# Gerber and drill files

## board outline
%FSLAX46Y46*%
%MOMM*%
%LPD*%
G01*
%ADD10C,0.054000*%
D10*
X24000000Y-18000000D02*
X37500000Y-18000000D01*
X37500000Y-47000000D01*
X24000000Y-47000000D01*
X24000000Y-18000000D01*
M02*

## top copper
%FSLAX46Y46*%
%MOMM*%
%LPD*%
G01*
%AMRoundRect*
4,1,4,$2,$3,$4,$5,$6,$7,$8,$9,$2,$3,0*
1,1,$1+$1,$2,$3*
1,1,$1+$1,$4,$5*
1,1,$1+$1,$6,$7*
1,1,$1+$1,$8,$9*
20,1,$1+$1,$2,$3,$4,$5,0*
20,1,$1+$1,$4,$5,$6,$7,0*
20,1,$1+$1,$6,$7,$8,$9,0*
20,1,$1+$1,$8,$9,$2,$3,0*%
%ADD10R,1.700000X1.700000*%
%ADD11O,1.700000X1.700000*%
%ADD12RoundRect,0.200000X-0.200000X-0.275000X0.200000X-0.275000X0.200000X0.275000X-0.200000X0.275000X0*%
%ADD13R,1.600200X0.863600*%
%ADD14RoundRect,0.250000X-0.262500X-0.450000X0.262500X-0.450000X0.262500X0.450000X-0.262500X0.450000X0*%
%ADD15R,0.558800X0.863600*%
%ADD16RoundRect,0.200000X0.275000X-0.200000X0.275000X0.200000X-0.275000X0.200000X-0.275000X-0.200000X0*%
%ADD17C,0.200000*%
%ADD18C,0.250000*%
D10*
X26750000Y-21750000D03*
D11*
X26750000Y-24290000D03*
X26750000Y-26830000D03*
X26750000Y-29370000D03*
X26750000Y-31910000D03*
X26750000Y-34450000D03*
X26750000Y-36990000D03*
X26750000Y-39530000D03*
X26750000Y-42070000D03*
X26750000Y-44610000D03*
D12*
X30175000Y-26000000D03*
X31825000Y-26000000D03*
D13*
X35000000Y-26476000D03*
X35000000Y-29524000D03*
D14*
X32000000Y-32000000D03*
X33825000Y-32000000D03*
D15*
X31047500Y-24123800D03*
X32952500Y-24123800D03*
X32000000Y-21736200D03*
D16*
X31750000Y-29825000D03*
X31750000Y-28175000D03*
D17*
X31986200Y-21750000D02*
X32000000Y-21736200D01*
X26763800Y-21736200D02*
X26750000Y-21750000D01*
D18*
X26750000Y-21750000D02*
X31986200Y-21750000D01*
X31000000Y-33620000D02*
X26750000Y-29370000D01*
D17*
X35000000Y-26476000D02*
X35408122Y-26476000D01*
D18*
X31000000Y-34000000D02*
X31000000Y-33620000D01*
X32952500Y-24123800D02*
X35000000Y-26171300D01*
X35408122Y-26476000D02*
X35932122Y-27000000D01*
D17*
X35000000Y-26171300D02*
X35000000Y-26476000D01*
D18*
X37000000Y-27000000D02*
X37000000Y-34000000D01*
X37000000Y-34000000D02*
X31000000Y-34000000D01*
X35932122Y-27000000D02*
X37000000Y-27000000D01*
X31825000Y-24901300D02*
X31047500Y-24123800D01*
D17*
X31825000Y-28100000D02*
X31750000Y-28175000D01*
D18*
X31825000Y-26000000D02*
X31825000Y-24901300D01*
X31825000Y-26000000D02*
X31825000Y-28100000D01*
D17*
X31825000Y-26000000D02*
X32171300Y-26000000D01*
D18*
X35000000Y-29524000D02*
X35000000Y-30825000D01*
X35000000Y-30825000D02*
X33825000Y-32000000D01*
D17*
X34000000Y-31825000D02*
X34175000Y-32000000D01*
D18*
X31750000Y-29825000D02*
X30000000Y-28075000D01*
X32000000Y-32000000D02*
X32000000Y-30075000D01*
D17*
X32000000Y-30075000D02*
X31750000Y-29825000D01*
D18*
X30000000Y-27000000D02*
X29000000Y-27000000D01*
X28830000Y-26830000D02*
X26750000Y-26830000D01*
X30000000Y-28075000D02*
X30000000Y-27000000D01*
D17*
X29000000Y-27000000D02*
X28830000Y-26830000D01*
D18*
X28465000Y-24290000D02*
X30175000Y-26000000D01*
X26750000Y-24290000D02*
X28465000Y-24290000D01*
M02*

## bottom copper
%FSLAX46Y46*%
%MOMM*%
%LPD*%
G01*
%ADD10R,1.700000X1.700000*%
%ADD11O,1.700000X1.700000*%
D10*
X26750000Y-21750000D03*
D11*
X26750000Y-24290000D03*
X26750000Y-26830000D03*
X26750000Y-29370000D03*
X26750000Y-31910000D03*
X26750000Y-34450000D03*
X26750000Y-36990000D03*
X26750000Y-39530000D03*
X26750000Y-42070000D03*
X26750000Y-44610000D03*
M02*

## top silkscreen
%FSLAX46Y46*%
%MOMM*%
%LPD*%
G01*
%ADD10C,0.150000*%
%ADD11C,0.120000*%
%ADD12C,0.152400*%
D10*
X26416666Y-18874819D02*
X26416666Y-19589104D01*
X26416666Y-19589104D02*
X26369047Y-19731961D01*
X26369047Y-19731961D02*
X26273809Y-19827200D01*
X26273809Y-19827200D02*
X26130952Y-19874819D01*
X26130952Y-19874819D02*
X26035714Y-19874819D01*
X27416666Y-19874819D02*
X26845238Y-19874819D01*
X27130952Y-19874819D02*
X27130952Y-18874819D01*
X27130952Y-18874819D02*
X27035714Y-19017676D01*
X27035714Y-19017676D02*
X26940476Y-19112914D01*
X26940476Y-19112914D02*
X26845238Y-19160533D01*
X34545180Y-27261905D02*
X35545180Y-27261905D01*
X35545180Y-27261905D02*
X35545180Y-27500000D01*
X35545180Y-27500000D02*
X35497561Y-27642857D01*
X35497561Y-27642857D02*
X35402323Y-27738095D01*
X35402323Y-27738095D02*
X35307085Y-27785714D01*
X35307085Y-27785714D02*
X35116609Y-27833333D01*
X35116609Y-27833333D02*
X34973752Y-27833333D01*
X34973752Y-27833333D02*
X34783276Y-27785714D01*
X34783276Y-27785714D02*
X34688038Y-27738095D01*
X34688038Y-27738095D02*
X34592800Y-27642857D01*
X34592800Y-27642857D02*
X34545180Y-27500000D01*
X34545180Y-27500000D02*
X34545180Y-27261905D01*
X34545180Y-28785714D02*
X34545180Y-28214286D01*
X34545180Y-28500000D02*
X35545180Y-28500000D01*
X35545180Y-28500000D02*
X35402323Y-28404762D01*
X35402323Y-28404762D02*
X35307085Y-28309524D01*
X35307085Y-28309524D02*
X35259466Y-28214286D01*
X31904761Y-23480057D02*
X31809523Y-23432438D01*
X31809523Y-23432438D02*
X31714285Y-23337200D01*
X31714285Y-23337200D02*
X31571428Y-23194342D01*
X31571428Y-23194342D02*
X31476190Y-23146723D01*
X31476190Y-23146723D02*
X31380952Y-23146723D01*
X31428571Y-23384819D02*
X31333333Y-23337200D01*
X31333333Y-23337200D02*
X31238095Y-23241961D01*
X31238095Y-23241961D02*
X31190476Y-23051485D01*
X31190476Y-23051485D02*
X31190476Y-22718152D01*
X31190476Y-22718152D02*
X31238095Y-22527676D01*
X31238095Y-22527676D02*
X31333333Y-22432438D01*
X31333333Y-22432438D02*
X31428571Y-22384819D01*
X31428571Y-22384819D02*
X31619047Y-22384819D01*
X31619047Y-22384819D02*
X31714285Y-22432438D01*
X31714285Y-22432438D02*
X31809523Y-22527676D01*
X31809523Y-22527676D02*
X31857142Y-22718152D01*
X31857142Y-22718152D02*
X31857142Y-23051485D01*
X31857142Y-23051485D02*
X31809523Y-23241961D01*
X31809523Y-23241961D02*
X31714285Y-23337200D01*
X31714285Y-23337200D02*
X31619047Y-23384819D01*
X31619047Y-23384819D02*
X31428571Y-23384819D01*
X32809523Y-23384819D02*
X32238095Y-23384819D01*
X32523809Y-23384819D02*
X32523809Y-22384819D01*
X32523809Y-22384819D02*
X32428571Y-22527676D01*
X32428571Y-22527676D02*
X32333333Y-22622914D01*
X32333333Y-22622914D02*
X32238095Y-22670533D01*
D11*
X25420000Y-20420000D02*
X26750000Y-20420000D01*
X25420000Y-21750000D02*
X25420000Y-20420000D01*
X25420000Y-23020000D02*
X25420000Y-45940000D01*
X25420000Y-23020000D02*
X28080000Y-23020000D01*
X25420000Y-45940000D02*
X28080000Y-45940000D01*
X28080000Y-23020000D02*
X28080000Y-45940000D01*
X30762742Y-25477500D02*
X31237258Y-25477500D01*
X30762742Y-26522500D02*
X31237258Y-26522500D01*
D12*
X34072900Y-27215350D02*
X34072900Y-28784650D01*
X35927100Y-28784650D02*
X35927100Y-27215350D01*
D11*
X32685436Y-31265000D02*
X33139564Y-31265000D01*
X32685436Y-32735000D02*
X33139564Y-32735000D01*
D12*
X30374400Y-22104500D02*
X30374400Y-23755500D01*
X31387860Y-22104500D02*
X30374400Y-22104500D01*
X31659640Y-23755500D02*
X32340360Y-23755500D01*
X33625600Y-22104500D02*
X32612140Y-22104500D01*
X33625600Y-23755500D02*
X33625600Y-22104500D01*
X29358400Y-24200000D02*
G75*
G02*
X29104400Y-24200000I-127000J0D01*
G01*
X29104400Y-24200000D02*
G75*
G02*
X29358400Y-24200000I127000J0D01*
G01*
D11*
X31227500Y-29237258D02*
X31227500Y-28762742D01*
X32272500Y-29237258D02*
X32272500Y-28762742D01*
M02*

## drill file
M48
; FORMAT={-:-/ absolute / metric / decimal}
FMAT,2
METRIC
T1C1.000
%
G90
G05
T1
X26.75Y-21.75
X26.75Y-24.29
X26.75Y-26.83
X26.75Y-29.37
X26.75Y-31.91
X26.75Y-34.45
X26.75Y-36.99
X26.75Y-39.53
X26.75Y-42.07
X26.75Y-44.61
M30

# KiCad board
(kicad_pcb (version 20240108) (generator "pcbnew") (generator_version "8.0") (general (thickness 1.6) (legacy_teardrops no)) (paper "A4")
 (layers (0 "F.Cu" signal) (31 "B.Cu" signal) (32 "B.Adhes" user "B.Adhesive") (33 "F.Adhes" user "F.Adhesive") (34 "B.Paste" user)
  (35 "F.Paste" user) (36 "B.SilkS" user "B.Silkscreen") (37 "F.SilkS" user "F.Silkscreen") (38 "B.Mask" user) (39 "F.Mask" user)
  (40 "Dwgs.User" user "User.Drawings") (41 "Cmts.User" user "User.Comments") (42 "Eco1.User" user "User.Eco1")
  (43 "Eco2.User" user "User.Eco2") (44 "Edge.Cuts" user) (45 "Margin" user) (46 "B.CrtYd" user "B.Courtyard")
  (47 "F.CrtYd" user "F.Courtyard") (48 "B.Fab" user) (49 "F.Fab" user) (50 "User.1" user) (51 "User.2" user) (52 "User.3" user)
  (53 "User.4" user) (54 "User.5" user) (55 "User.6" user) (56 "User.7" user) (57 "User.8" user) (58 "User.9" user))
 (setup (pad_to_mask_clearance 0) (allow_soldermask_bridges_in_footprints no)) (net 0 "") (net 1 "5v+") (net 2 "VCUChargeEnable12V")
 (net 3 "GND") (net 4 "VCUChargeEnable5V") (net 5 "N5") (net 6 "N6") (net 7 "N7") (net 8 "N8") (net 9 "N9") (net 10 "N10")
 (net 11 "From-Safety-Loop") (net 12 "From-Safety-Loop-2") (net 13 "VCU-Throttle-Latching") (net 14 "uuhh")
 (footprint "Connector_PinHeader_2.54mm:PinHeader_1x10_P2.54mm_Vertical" (layer "F.Cu") (at 26.75 21.75)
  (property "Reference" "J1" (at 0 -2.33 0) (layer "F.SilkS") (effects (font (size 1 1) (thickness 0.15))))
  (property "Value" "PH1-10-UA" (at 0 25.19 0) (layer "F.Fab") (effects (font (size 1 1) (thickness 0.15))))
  (fp_line (start -1.33 -1.33) (end 0 -1.33) (stroke (width 0.12) (type solid)) (layer "F.SilkS"))
  (fp_line (start -1.33 0) (end -1.33 -1.33) (stroke (width 0.12) (type solid)) (layer "F.SilkS"))
  (fp_line (start -1.33 1.27) (end -1.33 24.19) (stroke (width 0.12) (type solid)) (layer "F.SilkS"))
  (fp_line (start -1.33 1.27) (end 1.33 1.27) (stroke (width 0.12) (type solid)) (layer "F.SilkS"))
  (fp_line (start -1.33 24.19) (end 1.33 24.19) (stroke (width 0.12) (type solid)) (layer "F.SilkS"))
  (fp_line (start 1.33 1.27) (end 1.33 24.19) (stroke (width 0.12) (type solid)) (layer "F.SilkS"))
  (pad "1" thru_hole rect (at 0 0) (size 1.7 1.7) (drill 1) (layers "*.Cu" "*.Mask") (remove_unused_layers no) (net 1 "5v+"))
  (pad "2" thru_hole oval (at 0 2.54) (size 1.7 1.7) (drill 1) (layers "*.Cu" "*.Mask") (remove_unused_layers no)
   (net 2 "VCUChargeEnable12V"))
  (pad "3" thru_hole oval (at 0 5.08) (size 1.7 1.7) (drill 1) (layers "*.Cu" "*.Mask") (remove_unused_layers no) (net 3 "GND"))
  (pad "4" thru_hole oval (at 0 7.62) (size 1.7 1.7) (drill 1) (layers "*.Cu" "*.Mask") (remove_unused_layers no)
   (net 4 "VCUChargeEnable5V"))
  (pad "5" thru_hole oval (at 0 10.16) (size 1.7 1.7) (drill 1) (layers "*.Cu" "*.Mask") (remove_unused_layers no) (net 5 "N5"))
  (pad "6" thru_hole oval (at 0 12.7) (size 1.7 1.7) (drill 1) (layers "*.Cu" "*.Mask") (remove_unused_layers no) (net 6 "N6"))
  (pad "7" thru_hole oval (at 0 15.24) (size 1.7 1.7) (drill 1) (layers "*.Cu" "*.Mask") (remove_unused_layers no) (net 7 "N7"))
  (pad "8" thru_hole oval (at 0 17.78) (size 1.7 1.7) (drill 1) (layers "*.Cu" "*.Mask") (remove_unused_layers no) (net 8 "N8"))
  (pad "9" thru_hole oval (at 0 20.32) (size 1.7 1.7) (drill 1) (layers "*.Cu" "*.Mask") (remove_unused_layers no) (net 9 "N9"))
  (pad "10" thru_hole oval (at 0 22.86) (size 1.7 1.7) (drill 1) (layers "*.Cu" "*.Mask") (remove_unused_layers no) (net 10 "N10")))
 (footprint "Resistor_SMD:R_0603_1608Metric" (layer "F.Cu") (at 31 26)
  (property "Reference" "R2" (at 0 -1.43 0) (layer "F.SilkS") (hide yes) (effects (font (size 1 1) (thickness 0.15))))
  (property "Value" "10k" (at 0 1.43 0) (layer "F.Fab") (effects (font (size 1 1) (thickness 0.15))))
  (fp_line (start -0.237258 -0.5225) (end 0.237258 -0.5225) (stroke (width 0.12) (type solid)) (layer "F.SilkS"))
  (fp_line (start -0.237258 0.5225) (end 0.237258 0.5225) (stroke (width 0.12) (type solid)) (layer "F.SilkS"))
  (pad "1" smd roundrect (at -0.825 0) (size 0.8 0.95) (layers "F.Cu" "F.Paste" "F.Mask") (roundrect_rratio 0.25)
   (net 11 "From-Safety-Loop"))
  (pad "2" smd roundrect (at 0.825 0) (size 0.8 0.95) (layers "F.Cu" "F.Paste" "F.Mask") (roundrect_rratio 0.25)
   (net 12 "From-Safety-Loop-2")))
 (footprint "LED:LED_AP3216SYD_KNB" (layer "F.Cu") (at 35 28 -90)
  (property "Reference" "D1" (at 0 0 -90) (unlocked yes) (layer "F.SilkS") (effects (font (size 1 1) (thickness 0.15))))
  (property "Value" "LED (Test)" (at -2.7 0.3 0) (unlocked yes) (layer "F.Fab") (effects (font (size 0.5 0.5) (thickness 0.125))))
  (fp_line (start -0.78465 0.9271) (end 0.78465 0.9271) (stroke (width 0.1524) (type solid)) (layer "F.SilkS"))
  (fp_line (start 0.78465 -0.9271) (end -0.78465 -0.9271) (stroke (width 0.1524) (type solid)) (layer "F.SilkS"))
  (pad "1" smd rect (at -1.524 0 270) (size 0.8636 1.6002) (layers "F.Cu" "F.Paste" "F.Mask") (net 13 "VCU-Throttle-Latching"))
  (pad "2" smd rect (at 1.524 0 270) (size 0.8636 1.6002) (layers "F.Cu" "F.Paste" "F.Mask") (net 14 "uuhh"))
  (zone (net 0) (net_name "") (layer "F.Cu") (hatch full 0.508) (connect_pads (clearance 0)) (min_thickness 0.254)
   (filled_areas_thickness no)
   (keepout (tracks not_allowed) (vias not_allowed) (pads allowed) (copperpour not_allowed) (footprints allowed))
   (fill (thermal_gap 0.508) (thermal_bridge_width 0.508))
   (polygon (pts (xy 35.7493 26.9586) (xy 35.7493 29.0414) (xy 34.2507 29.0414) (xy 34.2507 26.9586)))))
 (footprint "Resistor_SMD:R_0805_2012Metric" (layer "F.Cu") (at 32.9125 32)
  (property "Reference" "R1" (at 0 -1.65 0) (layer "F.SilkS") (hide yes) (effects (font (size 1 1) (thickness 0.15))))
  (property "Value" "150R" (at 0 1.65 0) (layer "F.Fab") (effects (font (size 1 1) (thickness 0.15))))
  (fp_line (start -0.227064 -0.735) (end 0.227064 -0.735) (stroke (width 0.12) (type solid)) (layer "F.SilkS"))
  (fp_line (start -0.227064 0.735) (end 0.227064 0.735) (stroke (width 0.12) (type solid)) (layer "F.SilkS"))
  (pad "1" smd roundrect (at -0.9125 0) (size 1.025 1.4) (layers "F.Cu" "F.Paste" "F.Mask") (roundrect_rratio 0.243902) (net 3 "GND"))
  (pad "2" smd roundrect (at 0.9125 0) (size 1.025 1.4) (layers "F.Cu" "F.Paste" "F.Mask") (roundrect_rratio 0.243902) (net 14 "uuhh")))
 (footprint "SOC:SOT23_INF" (layer "F.Cu") (at 32 22.93)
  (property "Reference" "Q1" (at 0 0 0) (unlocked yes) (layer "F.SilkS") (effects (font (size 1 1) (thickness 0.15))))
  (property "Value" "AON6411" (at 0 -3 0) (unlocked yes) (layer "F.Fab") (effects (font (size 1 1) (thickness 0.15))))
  (fp_line (start -1.6256 -0.8255) (end -1.6256 0.8255) (stroke (width 0.1524) (type solid)) (layer "F.SilkS"))
  (fp_line (start -0.61214 -0.8255) (end -1.6256 -0.8255) (stroke (width 0.1524) (type solid)) (layer "F.SilkS"))
  (fp_line (start -0.34036 0.8255) (end 0.34036 0.8255) (stroke (width 0.1524) (type solid)) (layer "F.SilkS"))
  (fp_line (start 1.6256 -0.8255) (end 0.61214 -0.8255) (stroke (width 0.1524) (type solid)) (layer "F.SilkS"))
  (fp_line (start 1.6256 0.8255) (end 1.6256 -0.8255) (stroke (width 0.1524) (type solid)) (layer "F.SilkS"))
  (fp_circle (center -2.7686 1.27) (end -2.6416 1.27) (stroke (width 0.1524) (type solid)) (fill none) (layer "F.SilkS"))
  (pad "1" smd rect (at -0.9525 1.1938) (size 0.5588 0.8636) (layers "F.Cu" "F.Paste" "F.Mask") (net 12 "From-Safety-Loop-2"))
  (pad "2" smd rect (at 0.9525 1.1938) (size 0.5588 0.8636) (layers "F.Cu" "F.Paste" "F.Mask") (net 13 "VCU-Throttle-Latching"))
  (pad "3" smd rect (at 0 -1.1938) (size 0.5588 0.8636) (layers "F.Cu" "F.Paste" "F.Mask") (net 1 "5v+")))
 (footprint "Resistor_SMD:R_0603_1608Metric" (layer "F.Cu") (at 31.75 29 90)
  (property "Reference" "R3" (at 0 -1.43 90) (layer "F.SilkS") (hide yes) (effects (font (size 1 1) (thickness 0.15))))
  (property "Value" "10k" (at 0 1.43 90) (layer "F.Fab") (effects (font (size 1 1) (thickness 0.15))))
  (fp_line (start -0.237258 -0.5225) (end 0.237258 -0.5225) (stroke (width 0.12) (type solid)) (layer "F.SilkS"))
  (fp_line (start -0.237258 0.5225) (end 0.237258 0.5225) (stroke (width 0.12) (type solid)) (layer "F.SilkS"))
  (pad "1" smd roundrect (at -0.825 0 90) (size 0.8 0.95) (layers "F.Cu" "F.Paste" "F.Mask") (roundrect_rratio 0.25) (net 3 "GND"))
  (pad "2" smd roundrect (at 0.825 0 90) (size 0.8 0.95) (layers "F.Cu" "F.Paste" "F.Mask") (roundrect_rratio 0.25)
   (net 12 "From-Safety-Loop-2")))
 (gr_rect (start 24 18) (end 37.5 47) (stroke (width 0.054) (type default)) (fill none) (layer "Edge.Cuts"))
 (segment (start 31.9862 21.75) (end 32 21.7362) (width 0.2) (layer "F.Cu") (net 1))
 (segment (start 26.7638 21.7362) (end 26.75 21.75) (width 0.2) (layer "F.Cu") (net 1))
 (segment (start 26.75 21.75) (end 31.9862 21.75) (width 0.25) (layer "F.Cu") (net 1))
 (segment (start 31 33.62) (end 26.75 29.37) (width 0.25) (layer "F.Cu") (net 13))
 (segment (start 35 26.476) (end 35.408122 26.476) (width 0.2) (layer "F.Cu") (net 13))
 (segment (start 31 34) (end 31 33.62) (width 0.25) (layer "F.Cu") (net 13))
 (segment (start 32.9525 24.1238) (end 35 26.1713) (width 0.25) (layer "F.Cu") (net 13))
 (segment (start 35.408122 26.476) (end 35.932122 27) (width 0.25) (layer "F.Cu") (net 13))
 (segment (start 35 26.1713) (end 35 26.476) (width 0.2) (layer "F.Cu") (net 13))
 (segment (start 37 27) (end 37 34) (width 0.25) (layer "F.Cu") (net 13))
 (segment (start 37 34) (end 31 34) (width 0.25) (layer "F.Cu") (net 13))
 (segment (start 35.932122 27) (end 37 27) (width 0.25) (layer "F.Cu") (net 13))
 (segment (start 31.825 24.9013) (end 31.0475 24.1238) (width 0.25) (layer "F.Cu") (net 12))
 (segment (start 31.825 28.1) (end 31.75 28.175) (width 0.2) (layer "F.Cu") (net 12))
 (segment (start 31.825 26) (end 31.825 24.9013) (width 0.25) (layer "F.Cu") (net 12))
 (segment (start 31.825 26) (end 31.825 28.1) (width 0.25) (layer "F.Cu") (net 12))
 (segment (start 31.825 26) (end 32.1713 26) (width 0.2) (layer "F.Cu") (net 12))
 (segment (start 35 29.524) (end 35 30.825) (width 0.25) (layer "F.Cu") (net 14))
 (segment (start 35 30.825) (end 33.825 32) (width 0.25) (layer "F.Cu") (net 14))
 (segment (start 34 31.825) (end 34.175 32) (width 0.2) (layer "F.Cu") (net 14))
 (segment (start 31.75 29.825) (end 30 28.075) (width 0.25) (layer "F.Cu") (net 3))
 (segment (start 32 32) (end 32 30.075) (width 0.25) (layer "F.Cu") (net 3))
 (segment (start 32 30.075) (end 31.75 29.825) (width 0.2) (layer "F.Cu") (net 3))
 (segment (start 30 27) (end 29 27) (width 0.25) (layer "F.Cu") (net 3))
 (segment (start 28.83 26.83) (end 26.75 26.83) (width 0.25) (layer "F.Cu") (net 3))
 (segment (start 30 28.075) (end 30 27) (width 0.25) (layer "F.Cu") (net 3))
 (segment (start 29 27) (end 28.83 26.83) (width 0.2) (layer "F.Cu") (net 3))
 (segment (start 28.465 24.29) (end 30.175 26) (width 0.25) (layer "F.Cu") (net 11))
 (segment (start 26.75 24.29) (end 28.465 24.29) (width 0.25) (layer "F.Cu") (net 11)))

